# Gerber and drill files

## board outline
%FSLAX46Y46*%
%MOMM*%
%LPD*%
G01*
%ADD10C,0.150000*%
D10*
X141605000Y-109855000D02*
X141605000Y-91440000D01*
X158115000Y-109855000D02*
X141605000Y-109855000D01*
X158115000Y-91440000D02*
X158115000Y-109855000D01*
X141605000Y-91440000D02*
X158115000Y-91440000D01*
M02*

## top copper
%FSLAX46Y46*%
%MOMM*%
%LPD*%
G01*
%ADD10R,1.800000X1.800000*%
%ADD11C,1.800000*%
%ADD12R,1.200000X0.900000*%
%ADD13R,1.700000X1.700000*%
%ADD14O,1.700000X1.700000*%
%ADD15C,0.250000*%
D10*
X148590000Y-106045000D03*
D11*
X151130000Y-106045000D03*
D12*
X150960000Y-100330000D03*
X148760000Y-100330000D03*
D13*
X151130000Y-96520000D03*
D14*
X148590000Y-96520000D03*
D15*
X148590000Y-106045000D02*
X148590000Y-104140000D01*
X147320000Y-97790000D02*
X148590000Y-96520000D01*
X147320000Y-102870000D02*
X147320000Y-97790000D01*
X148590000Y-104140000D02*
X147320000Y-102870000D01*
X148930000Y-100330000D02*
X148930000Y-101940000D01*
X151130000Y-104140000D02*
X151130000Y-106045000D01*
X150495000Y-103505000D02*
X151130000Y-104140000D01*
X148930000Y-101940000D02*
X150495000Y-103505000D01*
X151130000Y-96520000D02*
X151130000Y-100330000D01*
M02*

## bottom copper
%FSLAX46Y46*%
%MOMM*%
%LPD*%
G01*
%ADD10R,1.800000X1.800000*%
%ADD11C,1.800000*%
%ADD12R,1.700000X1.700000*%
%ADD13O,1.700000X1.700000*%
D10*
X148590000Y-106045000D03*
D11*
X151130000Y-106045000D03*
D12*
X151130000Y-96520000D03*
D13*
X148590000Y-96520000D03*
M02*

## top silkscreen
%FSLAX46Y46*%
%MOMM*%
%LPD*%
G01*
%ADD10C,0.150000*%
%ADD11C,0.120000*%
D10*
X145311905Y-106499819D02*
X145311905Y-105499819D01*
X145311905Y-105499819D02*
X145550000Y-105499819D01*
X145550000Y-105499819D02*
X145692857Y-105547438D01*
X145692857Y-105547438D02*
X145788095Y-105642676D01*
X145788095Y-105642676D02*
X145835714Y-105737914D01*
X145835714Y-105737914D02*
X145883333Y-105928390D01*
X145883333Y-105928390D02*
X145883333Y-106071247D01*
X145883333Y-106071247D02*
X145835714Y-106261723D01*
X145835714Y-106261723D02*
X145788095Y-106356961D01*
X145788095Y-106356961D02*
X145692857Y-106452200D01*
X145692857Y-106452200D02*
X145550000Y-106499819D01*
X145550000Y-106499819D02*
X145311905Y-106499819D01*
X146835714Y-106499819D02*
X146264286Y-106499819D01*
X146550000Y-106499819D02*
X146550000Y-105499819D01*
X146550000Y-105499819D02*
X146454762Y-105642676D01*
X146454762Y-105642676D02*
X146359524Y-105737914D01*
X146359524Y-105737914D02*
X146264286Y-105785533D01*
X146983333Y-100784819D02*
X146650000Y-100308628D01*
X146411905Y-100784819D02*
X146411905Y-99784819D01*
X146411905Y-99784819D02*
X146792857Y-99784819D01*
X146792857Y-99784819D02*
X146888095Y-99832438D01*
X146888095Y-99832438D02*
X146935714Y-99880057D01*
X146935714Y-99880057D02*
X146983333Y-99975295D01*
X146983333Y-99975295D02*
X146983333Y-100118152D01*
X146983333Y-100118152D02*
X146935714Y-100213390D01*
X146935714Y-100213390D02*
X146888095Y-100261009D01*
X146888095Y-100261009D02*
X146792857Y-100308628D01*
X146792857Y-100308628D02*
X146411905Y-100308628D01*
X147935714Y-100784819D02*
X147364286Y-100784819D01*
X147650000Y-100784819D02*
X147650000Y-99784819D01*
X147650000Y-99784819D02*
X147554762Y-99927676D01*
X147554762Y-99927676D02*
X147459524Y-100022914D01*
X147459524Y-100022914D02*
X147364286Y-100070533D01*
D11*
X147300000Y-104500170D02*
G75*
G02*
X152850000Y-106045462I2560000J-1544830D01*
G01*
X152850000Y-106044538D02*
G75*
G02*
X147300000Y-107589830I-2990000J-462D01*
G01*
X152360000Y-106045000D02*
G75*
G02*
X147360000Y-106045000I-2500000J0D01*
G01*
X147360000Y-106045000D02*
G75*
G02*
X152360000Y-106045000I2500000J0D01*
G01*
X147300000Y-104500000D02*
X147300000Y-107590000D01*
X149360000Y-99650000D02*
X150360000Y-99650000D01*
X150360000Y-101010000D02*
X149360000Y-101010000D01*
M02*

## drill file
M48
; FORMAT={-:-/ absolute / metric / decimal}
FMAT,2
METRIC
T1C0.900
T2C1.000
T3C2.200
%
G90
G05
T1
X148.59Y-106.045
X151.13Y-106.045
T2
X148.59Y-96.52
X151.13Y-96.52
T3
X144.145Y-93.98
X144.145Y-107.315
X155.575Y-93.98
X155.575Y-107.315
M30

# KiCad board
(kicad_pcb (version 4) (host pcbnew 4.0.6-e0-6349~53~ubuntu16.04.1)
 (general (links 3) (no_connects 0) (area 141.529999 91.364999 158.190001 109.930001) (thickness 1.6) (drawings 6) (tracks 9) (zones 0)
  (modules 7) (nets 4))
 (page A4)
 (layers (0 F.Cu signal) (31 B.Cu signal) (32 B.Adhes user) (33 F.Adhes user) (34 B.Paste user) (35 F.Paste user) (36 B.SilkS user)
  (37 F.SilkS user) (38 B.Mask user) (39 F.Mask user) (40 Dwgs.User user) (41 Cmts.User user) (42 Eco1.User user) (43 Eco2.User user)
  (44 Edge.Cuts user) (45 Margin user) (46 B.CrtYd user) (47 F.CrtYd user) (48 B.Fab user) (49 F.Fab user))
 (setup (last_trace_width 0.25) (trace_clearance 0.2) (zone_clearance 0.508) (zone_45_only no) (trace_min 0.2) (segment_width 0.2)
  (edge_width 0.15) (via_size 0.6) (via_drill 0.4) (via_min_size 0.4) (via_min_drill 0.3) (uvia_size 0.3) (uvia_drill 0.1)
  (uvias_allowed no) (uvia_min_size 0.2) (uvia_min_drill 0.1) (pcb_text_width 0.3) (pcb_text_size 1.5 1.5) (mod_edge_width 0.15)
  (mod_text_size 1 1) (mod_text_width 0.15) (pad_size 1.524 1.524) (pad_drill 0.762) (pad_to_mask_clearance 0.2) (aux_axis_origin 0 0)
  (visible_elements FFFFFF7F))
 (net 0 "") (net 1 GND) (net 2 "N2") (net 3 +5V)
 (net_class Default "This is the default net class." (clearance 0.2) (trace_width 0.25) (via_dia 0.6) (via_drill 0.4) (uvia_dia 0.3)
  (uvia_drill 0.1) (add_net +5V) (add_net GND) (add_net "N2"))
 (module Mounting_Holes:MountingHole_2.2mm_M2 (layer F.Cu) (at 155.575 107.315)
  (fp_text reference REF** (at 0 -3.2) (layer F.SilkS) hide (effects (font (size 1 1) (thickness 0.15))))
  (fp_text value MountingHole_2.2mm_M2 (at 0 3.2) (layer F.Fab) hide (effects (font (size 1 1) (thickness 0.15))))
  (pad 1 np_thru_hole circle (at 0 0) (size 2.2 2.2) (drill 2.2) (layers *.Cu *.Mask)))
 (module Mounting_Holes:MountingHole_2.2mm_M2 (layer F.Cu) (at 144.145 107.315)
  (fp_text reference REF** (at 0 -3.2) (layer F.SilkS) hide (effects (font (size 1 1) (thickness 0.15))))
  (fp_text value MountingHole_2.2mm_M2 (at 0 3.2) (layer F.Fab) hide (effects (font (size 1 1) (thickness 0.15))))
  (pad 1 np_thru_hole circle (at 0 0) (size 2.2 2.2) (drill 2.2) (layers *.Cu *.Mask)))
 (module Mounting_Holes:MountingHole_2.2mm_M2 (layer F.Cu) (at 144.145 93.98)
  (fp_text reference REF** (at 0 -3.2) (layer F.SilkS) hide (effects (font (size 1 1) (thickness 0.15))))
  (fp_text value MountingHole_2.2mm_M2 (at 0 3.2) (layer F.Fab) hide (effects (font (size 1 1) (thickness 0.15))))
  (pad 1 np_thru_hole circle (at 0 0) (size 2.2 2.2) (drill 2.2) (layers *.Cu *.Mask)))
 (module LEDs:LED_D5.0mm (layer F.Cu) (at 148.59 106.045)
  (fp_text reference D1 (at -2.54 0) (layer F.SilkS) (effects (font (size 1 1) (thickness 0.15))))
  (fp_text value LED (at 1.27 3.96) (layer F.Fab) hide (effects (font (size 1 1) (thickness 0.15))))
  (fp_arc (start 1.27 0) (end -1.29 -1.54483) (angle 148.9) (layer F.SilkS) (width 0.12))
  (fp_arc (start 1.27 0) (end -1.29 1.54483) (angle -148.9) (layer F.SilkS) (width 0.12))
  (fp_circle (center 1.27 0) (end 3.77 0) (layer F.SilkS) (width 0.12))
  (fp_line (start -1.29 -1.545) (end -1.29 1.545) (layer F.SilkS) (width 0.12))
  (pad 1 thru_hole rect (at 0 0) (size 1.8 1.8) (drill 0.9) (layers *.Cu *.Mask) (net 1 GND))
  (pad 2 thru_hole circle (at 2.54 0) (size 1.8 1.8) (drill 0.9) (layers *.Cu *.Mask) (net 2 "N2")))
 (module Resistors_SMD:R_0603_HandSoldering (layer F.Cu) (at 149.86 100.33 180)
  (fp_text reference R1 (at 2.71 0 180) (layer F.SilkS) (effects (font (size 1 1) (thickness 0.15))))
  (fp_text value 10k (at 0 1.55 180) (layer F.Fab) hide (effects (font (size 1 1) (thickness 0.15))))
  (fp_line (start 0.5 0.68) (end -0.5 0.68) (layer F.SilkS) (width 0.12))
  (fp_line (start -0.5 -0.68) (end 0.5 -0.68) (layer F.SilkS) (width 0.12))
  (pad 1 smd rect (at -1.1 0 180) (size 1.2 0.9) (layers F.Cu F.Paste F.Mask) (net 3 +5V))
  (pad 2 smd rect (at 1.1 0 180) (size 1.2 0.9) (layers F.Cu F.Paste F.Mask) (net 2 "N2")))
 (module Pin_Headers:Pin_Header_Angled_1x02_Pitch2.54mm (layer B.Cu) (at 151.13 96.52 90)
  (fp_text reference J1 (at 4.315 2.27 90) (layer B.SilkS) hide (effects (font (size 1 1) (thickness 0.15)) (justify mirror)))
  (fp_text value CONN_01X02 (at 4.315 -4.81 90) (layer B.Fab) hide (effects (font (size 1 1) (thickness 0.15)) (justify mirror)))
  (pad 1 thru_hole rect (at 0 0 90) (size 1.7 1.7) (drill 1) (layers *.Cu *.Mask) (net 3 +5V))
  (pad 2 thru_hole oval (at 0 -2.54 90) (size 1.7 1.7) (drill 1) (layers *.Cu *.Mask) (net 1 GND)))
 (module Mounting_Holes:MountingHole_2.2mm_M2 (layer F.Cu) (at 155.575 93.98)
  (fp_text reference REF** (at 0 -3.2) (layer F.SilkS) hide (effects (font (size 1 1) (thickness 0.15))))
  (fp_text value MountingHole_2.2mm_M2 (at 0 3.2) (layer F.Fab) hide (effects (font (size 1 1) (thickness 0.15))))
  (pad 1 np_thru_hole circle (at 0 0) (size 2.2 2.2) (drill 2.2) (layers *.Cu *.Mask)))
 (gr_line (start 141.605 109.855) (end 141.605 91.44) (layer Edge.Cuts) (width 0.15))
 (gr_line (start 158.115 109.855) (end 141.605 109.855) (layer Edge.Cuts) (width 0.15))
 (gr_line (start 158.115 91.44) (end 158.115 109.855) (layer Edge.Cuts) (width 0.15))
 (gr_line (start 141.605 91.44) (end 158.115 91.44) (layer Edge.Cuts) (width 0.15))
 (segment (start 148.59 106.045) (end 148.59 104.14) (width 0.25) (layer F.Cu) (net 1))
 (segment (start 147.32 97.79) (end 148.59 96.52) (width 0.25) (layer F.Cu) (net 1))
 (segment (start 147.32 102.87) (end 147.32 97.79) (width 0.25) (layer F.Cu) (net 1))
 (segment (start 148.59 104.14) (end 147.32 102.87) (width 0.25) (layer F.Cu) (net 1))
 (segment (start 148.93 100.33) (end 148.93 101.94) (width 0.25) (layer F.Cu) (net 2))
 (segment (start 151.13 104.14) (end 151.13 106.045) (width 0.25) (layer F.Cu) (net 2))
 (segment (start 150.495 103.505) (end 151.13 104.14) (width 0.25) (layer F.Cu) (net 2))
 (segment (start 148.93 101.94) (end 150.495 103.505) (width 0.25) (layer F.Cu) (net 2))
 (segment (start 151.13 96.52) (end 151.13 100.33) (width 0.25) (layer F.Cu) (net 3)))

